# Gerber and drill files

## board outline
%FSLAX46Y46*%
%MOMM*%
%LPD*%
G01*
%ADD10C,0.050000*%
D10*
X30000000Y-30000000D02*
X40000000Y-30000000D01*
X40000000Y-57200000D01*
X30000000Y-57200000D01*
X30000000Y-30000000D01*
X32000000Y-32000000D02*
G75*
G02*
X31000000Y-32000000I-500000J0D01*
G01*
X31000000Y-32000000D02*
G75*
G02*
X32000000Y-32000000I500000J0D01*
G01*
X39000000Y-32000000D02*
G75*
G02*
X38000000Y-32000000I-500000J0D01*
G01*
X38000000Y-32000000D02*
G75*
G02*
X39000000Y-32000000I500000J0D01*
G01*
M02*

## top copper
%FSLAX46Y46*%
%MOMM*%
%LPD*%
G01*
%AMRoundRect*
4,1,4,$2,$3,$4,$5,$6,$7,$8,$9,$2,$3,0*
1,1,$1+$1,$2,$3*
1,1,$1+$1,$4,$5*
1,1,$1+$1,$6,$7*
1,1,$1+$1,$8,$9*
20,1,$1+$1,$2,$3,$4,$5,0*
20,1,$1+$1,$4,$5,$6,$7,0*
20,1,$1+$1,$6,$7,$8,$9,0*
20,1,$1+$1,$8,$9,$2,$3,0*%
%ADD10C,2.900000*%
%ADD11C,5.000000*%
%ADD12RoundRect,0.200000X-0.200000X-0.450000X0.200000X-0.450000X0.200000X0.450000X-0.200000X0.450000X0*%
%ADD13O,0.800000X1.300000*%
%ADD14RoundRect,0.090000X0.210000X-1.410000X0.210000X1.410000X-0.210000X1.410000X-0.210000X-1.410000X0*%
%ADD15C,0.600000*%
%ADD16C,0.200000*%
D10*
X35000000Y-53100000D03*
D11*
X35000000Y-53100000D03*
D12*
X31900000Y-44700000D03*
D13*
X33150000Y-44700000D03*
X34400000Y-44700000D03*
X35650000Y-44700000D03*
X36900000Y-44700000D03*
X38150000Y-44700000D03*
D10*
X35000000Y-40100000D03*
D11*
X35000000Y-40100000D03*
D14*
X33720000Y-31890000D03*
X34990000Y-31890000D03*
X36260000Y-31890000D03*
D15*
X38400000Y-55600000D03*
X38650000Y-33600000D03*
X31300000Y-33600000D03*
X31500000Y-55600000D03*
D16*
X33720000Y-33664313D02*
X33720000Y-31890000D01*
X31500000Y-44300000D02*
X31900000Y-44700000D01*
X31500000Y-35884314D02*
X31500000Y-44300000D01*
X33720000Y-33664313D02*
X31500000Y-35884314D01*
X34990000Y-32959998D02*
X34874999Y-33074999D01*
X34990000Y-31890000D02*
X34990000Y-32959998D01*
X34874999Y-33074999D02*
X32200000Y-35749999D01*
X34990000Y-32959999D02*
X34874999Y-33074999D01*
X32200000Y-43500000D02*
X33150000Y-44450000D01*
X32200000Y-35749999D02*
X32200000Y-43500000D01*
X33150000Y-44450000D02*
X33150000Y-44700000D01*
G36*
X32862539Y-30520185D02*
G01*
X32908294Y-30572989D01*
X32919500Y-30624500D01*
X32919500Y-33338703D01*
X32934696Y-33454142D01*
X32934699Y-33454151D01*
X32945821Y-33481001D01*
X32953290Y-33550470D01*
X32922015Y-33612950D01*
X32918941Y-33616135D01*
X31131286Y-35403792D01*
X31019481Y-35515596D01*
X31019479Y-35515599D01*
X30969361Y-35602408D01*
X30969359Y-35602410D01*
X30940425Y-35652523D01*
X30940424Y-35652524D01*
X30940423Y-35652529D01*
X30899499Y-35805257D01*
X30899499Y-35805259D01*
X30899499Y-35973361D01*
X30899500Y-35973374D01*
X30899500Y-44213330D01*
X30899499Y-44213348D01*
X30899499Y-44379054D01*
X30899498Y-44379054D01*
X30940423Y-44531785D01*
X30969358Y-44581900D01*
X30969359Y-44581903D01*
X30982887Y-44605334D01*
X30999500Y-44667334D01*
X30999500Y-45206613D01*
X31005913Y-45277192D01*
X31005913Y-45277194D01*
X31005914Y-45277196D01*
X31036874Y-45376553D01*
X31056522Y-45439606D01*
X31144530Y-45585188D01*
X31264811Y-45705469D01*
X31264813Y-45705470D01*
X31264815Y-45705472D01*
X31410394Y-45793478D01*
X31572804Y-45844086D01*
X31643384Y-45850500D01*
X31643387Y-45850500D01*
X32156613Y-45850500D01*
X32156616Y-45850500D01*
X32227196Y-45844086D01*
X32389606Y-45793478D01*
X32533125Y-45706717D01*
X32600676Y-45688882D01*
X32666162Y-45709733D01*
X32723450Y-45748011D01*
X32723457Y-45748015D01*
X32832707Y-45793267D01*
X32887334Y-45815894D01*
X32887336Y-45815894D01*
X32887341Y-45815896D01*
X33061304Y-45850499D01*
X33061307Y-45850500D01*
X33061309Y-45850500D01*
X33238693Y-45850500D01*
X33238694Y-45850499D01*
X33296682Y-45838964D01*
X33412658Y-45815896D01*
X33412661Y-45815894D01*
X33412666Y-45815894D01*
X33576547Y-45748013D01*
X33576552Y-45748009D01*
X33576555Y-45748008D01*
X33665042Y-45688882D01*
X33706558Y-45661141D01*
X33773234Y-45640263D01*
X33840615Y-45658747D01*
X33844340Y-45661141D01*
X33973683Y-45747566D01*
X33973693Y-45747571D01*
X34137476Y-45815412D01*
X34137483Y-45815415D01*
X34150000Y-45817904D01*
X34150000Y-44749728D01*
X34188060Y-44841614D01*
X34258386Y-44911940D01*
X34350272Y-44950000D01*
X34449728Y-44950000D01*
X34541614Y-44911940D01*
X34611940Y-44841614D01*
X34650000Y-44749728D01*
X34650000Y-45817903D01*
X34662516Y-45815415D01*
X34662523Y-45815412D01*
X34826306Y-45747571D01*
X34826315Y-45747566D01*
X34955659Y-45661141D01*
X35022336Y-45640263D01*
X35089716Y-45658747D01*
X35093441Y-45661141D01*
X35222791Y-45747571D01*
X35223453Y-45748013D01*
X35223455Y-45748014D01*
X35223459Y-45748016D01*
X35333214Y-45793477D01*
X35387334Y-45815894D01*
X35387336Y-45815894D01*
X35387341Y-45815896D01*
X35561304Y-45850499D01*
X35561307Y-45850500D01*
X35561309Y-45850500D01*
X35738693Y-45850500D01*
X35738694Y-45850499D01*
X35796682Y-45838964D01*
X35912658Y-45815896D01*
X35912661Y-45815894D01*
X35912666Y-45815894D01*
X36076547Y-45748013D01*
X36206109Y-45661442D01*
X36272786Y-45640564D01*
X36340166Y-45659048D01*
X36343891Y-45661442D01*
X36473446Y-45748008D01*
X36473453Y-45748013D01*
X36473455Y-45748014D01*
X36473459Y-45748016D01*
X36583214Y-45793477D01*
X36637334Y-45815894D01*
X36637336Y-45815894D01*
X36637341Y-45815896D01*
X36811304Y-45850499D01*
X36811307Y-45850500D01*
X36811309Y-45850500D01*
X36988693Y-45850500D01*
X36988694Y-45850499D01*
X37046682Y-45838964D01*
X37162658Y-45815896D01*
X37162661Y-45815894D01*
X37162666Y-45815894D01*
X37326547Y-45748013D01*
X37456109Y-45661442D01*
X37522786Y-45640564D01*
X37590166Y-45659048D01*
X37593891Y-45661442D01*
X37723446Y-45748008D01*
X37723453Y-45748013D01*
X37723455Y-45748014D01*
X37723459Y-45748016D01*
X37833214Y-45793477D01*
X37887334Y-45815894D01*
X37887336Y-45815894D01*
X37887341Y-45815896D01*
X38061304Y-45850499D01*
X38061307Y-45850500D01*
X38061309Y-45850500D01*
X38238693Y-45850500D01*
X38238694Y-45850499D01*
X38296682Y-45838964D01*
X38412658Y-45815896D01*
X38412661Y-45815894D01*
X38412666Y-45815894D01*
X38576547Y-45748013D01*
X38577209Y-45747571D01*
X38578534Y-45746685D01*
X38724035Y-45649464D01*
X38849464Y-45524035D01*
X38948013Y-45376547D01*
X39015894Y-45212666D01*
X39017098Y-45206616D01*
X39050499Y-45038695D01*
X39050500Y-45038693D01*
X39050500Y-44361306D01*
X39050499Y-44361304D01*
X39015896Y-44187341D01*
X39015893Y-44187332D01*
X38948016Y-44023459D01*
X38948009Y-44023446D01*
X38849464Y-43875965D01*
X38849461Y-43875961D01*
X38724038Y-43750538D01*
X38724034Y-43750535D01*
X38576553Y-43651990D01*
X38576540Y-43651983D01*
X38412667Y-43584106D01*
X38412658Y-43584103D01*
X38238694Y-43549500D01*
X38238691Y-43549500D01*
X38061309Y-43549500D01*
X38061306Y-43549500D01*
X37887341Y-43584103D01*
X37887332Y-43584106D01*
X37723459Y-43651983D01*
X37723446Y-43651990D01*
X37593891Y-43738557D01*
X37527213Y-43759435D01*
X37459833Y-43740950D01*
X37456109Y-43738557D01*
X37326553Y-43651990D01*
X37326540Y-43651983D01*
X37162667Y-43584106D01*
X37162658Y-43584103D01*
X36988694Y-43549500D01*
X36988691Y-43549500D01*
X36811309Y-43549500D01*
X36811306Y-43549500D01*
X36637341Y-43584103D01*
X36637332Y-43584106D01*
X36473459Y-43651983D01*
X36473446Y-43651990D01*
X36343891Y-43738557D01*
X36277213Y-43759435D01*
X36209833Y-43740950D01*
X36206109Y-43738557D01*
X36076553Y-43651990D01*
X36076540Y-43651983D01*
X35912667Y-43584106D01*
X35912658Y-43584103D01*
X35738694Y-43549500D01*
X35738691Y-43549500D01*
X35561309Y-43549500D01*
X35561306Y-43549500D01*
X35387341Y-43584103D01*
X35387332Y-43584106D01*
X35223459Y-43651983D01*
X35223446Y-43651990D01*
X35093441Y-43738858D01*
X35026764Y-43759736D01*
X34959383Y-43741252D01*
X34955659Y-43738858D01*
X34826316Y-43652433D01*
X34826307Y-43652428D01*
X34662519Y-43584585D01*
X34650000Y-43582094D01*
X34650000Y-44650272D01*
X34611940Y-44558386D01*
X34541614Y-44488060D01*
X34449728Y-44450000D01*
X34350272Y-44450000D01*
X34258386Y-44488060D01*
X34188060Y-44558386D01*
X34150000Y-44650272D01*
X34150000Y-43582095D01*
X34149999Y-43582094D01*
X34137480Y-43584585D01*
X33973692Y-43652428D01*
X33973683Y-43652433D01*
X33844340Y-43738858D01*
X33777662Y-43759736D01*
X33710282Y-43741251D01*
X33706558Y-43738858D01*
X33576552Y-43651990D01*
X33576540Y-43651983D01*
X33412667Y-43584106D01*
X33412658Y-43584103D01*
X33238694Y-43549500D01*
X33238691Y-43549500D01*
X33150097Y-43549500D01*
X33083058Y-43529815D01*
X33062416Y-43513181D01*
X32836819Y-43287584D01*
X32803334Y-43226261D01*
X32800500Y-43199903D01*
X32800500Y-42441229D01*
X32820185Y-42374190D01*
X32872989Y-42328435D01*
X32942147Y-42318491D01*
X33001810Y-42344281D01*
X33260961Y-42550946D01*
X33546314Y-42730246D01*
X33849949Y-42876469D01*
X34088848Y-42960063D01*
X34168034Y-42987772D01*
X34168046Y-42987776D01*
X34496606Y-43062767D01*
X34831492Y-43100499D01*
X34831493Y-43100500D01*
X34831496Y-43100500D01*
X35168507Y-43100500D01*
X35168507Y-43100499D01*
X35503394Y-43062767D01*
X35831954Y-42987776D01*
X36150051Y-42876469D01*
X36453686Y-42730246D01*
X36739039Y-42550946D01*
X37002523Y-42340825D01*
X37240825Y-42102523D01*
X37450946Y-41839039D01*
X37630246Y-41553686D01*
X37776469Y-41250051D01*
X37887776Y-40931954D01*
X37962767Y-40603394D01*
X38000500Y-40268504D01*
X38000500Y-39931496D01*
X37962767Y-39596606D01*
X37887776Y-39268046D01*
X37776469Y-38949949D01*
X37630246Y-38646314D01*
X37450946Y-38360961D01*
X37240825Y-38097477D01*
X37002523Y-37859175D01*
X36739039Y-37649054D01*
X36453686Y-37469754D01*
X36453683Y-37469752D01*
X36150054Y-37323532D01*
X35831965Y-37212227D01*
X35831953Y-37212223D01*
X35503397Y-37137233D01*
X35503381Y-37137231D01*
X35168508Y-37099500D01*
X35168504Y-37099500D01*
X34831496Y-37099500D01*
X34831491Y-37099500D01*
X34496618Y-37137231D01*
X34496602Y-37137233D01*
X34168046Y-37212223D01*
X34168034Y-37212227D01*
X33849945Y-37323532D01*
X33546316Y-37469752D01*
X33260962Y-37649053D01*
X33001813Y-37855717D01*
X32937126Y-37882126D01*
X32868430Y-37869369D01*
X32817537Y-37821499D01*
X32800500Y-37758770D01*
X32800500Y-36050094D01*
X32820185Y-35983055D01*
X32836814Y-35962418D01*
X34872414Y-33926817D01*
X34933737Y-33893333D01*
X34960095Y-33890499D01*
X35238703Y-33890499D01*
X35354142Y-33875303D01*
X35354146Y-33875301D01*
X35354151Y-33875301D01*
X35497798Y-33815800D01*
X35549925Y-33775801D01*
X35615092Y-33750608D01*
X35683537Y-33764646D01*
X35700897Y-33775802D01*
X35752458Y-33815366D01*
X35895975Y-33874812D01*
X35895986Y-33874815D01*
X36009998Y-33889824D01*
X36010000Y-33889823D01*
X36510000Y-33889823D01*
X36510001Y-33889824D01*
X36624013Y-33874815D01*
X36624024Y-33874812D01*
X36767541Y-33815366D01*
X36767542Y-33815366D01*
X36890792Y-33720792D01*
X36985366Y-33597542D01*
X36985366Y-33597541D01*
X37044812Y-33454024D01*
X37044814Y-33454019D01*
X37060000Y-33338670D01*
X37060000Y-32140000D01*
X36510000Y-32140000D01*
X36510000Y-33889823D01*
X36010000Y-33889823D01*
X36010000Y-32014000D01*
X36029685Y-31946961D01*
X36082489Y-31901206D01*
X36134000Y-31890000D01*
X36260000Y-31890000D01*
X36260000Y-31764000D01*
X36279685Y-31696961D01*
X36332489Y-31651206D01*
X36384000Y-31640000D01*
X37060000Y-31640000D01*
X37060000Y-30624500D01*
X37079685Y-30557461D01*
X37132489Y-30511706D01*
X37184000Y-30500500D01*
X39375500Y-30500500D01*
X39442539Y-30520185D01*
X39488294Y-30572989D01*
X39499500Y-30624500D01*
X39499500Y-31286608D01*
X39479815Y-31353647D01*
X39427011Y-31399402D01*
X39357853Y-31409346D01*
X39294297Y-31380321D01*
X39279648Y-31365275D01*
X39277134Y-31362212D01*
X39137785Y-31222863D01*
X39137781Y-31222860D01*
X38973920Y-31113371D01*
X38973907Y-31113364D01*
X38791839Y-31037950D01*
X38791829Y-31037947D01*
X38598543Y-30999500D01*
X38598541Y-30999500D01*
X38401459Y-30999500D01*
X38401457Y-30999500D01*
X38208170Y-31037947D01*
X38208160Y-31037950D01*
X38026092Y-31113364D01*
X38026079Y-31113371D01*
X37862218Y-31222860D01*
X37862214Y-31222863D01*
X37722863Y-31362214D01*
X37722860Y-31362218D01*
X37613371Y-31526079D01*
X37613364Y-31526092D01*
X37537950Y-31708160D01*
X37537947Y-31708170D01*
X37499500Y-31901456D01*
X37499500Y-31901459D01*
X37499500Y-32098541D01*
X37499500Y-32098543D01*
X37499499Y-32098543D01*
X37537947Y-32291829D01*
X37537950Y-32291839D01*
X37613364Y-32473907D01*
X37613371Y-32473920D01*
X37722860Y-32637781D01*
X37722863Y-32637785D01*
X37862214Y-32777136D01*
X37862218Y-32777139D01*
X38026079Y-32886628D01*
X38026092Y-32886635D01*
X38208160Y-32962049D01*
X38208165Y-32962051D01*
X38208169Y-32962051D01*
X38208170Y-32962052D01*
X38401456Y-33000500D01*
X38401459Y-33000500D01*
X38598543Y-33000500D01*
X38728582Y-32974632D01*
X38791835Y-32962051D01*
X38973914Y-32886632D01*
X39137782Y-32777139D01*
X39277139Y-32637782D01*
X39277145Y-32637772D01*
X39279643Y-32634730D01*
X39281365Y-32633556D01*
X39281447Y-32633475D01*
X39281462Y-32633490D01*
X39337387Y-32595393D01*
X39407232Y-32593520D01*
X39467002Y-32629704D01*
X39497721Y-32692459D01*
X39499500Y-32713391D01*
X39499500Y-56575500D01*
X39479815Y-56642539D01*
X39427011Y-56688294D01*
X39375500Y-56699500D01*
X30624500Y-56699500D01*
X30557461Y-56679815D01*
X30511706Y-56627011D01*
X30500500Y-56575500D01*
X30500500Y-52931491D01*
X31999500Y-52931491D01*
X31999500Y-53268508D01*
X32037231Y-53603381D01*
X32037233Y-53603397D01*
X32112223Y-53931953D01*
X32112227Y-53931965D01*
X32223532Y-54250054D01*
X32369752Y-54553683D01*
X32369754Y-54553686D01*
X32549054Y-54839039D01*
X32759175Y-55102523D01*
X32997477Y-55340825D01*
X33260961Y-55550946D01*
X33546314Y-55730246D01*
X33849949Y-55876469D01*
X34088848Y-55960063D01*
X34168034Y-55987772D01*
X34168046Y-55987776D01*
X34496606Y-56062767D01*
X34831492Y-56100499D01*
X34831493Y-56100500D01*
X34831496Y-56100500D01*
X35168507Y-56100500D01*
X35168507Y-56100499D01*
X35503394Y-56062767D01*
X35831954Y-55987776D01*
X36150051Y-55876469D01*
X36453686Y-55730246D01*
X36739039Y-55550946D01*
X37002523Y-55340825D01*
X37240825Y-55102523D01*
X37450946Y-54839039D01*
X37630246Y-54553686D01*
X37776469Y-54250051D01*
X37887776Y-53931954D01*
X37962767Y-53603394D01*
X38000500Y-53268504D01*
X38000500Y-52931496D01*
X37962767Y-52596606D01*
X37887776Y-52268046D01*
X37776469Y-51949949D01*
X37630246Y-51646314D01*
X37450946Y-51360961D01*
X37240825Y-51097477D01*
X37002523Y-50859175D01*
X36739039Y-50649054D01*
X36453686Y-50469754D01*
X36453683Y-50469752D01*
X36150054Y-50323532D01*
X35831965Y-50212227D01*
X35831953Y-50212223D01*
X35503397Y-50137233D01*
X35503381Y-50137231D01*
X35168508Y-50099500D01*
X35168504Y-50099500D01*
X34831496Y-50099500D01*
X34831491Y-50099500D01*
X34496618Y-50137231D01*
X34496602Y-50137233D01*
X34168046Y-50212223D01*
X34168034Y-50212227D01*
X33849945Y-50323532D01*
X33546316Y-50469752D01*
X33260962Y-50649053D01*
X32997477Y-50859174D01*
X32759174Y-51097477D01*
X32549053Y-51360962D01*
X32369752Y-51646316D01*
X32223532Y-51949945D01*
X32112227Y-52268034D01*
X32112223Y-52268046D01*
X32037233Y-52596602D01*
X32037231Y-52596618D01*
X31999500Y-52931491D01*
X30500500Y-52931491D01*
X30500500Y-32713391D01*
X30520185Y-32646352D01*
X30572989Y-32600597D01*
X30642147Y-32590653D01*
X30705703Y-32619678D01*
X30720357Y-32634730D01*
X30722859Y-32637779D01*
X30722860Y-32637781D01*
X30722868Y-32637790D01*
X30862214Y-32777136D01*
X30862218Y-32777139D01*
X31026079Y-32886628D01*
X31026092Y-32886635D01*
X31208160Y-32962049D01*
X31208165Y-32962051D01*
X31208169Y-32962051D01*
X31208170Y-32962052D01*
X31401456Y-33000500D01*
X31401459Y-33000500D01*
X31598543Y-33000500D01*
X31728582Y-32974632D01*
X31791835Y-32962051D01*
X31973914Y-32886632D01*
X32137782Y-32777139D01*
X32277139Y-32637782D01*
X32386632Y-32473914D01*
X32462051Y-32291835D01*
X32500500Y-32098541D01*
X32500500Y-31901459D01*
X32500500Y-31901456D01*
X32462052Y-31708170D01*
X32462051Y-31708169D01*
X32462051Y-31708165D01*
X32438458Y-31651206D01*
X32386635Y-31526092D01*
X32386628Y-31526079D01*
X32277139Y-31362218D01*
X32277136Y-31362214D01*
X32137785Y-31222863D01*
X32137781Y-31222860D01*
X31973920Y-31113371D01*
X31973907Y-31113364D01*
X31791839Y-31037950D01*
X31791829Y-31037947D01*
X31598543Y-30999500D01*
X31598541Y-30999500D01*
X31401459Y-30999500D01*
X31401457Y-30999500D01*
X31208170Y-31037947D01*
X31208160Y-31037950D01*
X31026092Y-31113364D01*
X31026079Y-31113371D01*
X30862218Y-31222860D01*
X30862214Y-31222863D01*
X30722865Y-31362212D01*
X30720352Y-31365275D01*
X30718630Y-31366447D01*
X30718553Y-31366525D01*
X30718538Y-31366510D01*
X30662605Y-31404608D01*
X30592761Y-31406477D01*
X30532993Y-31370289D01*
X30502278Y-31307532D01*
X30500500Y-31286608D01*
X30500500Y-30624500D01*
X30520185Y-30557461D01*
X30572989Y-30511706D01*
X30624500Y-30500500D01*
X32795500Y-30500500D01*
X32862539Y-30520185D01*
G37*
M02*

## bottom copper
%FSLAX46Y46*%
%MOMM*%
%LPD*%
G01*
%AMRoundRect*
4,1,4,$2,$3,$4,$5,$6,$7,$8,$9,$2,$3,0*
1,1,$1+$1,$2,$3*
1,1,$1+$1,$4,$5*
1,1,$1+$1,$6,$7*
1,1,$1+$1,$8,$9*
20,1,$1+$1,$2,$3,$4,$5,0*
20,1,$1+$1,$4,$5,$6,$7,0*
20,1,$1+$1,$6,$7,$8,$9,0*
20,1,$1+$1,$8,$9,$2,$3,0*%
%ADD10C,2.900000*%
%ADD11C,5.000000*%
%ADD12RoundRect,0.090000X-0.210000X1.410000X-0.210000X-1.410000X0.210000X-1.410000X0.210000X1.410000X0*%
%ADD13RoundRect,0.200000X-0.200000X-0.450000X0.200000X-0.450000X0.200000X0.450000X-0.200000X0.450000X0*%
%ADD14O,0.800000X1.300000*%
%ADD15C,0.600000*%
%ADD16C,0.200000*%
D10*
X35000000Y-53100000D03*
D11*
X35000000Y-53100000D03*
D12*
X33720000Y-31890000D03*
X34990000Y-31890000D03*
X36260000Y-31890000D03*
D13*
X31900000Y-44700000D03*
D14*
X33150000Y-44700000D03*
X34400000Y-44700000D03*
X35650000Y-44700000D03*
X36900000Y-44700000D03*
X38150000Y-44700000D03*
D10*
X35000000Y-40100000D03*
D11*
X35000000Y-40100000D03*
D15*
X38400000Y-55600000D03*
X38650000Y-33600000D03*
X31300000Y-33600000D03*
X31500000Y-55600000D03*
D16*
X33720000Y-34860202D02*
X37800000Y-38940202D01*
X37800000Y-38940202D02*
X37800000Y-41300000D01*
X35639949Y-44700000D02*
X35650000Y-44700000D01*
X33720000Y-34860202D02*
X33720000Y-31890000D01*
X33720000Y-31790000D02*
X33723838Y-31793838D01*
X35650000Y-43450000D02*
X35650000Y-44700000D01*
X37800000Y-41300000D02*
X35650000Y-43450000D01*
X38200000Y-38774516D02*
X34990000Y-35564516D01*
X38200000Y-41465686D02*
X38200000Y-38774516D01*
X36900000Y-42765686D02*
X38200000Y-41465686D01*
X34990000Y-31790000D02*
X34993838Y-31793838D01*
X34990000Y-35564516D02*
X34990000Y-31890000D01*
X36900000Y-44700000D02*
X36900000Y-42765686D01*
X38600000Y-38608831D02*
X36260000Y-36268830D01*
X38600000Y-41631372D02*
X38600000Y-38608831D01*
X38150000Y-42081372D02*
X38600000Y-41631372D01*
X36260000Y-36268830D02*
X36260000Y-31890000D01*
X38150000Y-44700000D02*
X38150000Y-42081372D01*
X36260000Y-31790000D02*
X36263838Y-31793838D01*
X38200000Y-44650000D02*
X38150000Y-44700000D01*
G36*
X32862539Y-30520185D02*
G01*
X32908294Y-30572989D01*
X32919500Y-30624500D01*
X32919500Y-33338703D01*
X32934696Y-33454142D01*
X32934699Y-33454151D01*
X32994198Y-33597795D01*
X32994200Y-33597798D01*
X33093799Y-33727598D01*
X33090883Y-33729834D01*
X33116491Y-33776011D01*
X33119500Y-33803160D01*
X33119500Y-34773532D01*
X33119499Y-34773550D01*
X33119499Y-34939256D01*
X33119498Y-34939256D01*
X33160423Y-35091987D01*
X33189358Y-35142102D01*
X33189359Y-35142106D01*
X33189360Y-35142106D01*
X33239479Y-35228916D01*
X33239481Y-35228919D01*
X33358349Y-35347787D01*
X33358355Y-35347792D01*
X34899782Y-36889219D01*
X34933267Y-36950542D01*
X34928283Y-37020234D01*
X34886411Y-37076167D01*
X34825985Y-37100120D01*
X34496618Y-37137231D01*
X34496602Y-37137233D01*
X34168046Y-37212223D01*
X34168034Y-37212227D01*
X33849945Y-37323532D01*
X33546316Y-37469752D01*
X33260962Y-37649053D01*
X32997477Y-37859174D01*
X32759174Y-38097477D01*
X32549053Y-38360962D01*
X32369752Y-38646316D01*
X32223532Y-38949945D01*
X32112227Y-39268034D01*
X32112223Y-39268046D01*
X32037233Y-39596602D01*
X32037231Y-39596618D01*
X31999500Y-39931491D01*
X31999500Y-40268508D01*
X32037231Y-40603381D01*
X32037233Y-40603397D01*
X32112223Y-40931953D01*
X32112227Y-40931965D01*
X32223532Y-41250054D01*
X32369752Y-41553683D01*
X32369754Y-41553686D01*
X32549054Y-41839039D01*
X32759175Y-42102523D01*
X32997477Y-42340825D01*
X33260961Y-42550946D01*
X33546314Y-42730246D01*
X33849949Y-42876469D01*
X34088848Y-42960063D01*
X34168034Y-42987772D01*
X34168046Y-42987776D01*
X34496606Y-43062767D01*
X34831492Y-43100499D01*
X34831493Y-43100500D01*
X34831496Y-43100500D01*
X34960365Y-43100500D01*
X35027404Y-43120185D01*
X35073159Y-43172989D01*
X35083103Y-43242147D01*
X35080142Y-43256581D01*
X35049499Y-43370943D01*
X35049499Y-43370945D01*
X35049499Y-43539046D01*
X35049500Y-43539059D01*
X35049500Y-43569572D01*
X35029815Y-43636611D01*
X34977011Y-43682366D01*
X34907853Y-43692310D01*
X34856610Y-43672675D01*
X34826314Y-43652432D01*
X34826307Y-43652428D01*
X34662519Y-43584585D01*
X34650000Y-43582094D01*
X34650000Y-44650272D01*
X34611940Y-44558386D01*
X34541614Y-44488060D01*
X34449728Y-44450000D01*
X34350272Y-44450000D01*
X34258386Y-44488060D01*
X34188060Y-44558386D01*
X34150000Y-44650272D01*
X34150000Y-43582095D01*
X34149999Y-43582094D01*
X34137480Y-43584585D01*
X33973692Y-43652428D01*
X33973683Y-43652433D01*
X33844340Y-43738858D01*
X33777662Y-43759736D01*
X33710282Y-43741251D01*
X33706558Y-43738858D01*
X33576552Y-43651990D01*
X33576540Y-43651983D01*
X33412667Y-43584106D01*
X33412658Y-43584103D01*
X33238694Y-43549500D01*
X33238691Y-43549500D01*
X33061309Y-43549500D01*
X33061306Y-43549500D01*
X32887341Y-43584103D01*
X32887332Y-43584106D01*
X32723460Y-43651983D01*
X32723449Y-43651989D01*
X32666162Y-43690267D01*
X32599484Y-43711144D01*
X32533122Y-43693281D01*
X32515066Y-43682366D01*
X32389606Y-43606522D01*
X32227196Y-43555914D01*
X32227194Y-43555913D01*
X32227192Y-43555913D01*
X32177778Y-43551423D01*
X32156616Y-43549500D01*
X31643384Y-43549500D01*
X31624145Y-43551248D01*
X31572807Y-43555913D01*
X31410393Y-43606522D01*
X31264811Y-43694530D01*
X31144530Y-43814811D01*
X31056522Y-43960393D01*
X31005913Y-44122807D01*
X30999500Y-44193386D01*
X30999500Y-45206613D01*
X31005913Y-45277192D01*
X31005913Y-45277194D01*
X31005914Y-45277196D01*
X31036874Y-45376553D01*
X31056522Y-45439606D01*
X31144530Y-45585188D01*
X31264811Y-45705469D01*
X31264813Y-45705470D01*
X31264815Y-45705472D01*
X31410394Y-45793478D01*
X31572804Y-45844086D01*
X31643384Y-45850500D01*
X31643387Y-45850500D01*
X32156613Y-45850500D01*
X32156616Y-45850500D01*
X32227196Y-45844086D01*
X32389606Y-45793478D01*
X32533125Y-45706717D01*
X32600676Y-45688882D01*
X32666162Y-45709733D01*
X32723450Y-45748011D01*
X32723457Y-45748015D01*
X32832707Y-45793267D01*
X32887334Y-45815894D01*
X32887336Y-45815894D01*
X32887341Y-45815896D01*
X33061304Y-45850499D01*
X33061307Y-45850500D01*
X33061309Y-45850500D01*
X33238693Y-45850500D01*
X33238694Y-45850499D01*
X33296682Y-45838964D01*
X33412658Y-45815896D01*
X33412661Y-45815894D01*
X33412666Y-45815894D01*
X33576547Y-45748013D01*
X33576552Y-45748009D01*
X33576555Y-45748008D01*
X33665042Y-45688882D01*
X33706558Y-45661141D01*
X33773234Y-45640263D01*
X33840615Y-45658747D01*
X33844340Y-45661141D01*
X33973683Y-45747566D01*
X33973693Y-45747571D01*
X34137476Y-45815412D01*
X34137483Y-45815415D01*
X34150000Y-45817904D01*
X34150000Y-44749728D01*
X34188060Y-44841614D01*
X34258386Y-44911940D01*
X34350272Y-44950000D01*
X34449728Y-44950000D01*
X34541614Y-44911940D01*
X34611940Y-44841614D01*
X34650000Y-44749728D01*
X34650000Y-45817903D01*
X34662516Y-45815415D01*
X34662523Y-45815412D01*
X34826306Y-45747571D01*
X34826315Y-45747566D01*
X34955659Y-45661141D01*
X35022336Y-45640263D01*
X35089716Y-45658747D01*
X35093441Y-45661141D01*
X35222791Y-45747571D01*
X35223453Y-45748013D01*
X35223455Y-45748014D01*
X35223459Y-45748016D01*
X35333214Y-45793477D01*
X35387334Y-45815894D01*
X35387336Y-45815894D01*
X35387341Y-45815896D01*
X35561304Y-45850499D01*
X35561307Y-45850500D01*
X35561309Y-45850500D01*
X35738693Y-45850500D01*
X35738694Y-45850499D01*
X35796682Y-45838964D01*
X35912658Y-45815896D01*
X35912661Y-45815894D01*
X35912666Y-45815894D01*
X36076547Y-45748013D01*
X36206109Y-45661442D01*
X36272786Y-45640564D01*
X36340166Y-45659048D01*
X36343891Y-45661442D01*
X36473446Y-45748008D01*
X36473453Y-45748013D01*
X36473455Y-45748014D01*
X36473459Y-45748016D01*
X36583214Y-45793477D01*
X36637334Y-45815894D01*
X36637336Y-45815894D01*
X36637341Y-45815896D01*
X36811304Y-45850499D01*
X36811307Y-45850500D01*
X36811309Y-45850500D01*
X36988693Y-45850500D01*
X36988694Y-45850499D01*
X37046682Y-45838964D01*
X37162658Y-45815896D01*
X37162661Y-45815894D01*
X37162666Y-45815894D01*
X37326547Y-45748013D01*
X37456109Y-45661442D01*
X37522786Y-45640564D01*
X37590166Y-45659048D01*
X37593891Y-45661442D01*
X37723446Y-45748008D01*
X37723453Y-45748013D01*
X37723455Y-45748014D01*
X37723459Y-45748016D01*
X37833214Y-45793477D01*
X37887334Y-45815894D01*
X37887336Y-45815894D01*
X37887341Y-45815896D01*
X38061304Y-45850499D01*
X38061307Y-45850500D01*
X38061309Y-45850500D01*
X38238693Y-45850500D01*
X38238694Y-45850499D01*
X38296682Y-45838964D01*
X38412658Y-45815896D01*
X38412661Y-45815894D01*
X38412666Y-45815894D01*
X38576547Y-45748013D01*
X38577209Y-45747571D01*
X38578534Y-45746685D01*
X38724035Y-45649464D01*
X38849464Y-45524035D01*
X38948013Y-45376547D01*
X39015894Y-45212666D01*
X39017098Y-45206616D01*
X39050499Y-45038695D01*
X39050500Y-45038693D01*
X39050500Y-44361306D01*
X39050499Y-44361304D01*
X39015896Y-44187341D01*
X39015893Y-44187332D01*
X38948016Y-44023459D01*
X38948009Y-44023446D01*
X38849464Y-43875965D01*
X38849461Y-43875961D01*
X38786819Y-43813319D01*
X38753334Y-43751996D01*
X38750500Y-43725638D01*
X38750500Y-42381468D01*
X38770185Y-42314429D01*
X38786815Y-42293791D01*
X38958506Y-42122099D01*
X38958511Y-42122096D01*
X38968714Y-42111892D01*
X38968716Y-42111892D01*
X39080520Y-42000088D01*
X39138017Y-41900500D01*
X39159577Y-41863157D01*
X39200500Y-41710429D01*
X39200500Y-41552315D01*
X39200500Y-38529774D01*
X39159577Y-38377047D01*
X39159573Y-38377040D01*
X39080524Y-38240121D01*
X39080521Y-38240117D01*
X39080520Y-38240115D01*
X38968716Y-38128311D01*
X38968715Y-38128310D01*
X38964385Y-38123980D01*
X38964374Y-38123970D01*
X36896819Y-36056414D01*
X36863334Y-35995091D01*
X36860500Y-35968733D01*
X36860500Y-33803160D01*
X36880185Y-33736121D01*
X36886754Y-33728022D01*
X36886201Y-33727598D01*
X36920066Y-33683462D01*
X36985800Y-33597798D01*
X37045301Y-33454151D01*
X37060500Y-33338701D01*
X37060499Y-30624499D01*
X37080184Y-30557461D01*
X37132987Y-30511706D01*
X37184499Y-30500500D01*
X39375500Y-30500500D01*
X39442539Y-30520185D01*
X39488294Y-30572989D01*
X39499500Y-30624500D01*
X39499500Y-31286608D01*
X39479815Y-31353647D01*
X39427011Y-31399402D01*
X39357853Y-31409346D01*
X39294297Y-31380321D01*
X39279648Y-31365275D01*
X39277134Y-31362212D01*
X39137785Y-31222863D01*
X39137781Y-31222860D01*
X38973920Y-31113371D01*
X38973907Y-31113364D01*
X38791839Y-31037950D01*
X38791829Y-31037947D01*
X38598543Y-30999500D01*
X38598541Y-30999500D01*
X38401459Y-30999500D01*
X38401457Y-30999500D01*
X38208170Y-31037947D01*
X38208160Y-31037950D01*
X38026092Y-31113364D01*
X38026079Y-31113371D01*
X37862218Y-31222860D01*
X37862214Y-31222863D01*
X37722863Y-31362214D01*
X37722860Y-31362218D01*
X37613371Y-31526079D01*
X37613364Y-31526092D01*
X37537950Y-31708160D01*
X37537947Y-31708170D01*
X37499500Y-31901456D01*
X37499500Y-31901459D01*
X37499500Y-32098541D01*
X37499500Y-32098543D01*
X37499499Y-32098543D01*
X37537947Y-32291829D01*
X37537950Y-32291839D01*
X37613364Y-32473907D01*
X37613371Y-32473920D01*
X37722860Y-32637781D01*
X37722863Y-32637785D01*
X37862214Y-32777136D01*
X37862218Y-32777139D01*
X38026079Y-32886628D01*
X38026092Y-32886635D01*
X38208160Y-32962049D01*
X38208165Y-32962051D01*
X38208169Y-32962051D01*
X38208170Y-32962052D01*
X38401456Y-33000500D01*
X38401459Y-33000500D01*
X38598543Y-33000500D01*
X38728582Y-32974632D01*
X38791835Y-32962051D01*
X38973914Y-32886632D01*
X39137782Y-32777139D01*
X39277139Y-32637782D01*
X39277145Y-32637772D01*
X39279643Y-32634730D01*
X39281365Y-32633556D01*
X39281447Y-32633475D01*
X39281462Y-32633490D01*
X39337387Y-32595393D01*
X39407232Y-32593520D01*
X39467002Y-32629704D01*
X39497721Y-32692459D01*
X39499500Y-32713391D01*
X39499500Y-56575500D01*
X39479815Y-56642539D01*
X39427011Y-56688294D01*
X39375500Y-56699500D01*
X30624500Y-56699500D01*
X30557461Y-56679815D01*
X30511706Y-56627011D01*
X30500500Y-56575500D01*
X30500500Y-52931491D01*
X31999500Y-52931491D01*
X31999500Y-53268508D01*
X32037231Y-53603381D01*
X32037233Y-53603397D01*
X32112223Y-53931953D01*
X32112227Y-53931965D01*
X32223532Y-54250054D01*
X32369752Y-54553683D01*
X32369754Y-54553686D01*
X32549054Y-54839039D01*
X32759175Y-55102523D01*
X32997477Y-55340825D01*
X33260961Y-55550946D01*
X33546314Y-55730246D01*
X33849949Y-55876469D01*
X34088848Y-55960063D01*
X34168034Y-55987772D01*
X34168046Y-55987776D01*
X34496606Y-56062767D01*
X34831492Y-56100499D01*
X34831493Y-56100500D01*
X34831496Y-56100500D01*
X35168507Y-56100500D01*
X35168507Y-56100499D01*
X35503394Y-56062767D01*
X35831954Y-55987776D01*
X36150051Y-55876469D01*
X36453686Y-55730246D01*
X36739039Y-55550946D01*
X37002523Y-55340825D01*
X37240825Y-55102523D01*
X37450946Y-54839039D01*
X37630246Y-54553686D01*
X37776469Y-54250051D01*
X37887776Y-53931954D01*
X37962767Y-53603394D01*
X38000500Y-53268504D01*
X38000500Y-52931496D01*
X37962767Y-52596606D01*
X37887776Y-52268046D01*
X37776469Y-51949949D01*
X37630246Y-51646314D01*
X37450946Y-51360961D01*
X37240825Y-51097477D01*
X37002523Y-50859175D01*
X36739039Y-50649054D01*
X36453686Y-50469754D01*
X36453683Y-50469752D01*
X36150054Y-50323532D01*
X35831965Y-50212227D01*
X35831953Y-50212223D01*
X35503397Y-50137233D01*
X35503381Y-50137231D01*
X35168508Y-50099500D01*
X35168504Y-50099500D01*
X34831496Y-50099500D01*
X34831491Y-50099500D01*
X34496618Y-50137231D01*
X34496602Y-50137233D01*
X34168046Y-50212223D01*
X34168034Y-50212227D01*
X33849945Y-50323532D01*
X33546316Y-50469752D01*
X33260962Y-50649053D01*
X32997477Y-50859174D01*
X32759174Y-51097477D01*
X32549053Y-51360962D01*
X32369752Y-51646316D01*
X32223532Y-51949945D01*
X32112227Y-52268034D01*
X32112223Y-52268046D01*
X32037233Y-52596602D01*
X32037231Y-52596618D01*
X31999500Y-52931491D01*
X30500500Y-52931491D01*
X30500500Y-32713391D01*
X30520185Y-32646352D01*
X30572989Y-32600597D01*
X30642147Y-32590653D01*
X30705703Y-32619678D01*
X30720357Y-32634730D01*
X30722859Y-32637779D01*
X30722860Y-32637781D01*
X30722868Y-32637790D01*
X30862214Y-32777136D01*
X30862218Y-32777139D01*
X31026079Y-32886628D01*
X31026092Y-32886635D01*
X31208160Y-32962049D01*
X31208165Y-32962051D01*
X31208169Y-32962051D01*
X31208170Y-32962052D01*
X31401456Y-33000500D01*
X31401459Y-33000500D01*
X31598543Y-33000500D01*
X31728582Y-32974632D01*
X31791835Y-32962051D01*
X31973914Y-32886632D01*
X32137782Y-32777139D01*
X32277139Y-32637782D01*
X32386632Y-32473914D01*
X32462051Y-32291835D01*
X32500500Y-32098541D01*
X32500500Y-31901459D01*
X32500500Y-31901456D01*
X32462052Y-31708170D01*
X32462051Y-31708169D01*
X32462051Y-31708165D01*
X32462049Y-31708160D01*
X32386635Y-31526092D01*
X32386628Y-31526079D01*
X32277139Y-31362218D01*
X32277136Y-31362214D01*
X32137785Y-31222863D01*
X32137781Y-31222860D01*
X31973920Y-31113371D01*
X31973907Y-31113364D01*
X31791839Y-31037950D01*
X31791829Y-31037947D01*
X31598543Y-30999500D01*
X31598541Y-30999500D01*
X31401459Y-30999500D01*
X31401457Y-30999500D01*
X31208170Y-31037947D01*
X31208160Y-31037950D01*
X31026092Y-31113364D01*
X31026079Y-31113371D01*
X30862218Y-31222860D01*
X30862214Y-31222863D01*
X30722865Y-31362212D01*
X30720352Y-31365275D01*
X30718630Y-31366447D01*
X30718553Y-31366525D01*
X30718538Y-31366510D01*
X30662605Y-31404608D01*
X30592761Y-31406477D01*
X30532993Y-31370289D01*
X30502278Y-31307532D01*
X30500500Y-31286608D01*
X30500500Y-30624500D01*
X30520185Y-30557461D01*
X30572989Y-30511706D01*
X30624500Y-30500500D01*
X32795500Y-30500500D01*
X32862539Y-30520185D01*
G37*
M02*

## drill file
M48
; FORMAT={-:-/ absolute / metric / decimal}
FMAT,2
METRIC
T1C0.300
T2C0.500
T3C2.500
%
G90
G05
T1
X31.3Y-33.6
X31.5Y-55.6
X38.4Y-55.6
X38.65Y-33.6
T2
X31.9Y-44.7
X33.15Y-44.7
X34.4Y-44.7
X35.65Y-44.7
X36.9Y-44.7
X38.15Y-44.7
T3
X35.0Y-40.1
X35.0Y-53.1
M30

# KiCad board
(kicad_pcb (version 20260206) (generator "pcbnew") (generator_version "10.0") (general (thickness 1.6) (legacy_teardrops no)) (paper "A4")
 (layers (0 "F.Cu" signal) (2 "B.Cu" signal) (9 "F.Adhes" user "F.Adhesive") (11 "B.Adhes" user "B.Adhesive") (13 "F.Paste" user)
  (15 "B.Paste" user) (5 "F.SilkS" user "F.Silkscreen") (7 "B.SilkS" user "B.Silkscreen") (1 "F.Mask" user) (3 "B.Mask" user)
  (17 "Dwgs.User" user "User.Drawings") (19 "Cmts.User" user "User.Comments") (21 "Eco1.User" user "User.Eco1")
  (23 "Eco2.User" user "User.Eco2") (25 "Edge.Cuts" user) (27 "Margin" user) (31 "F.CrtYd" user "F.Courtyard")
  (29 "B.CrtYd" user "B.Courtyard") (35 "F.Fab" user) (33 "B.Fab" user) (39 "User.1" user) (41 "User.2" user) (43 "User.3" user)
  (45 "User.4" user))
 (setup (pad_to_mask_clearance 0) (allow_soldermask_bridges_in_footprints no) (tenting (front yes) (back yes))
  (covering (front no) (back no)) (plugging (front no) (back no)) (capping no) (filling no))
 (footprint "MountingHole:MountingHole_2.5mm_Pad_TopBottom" (layer "F.Cu") (at 35 53.1)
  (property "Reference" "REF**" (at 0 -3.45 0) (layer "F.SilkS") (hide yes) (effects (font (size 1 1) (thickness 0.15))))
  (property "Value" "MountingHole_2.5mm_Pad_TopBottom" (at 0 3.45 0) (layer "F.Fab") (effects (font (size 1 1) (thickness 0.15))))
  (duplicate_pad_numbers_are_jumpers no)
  (pad "1" thru_hole circle (at 0 0) (size 2.9 2.9) (drill 2.5) (layers "*.Cu" "*.Mask") (remove_unused_layers no) (zone_connect 2))
  (pad "1" connect circle (at 0 0) (size 5 5) (layers "F.Cu" "F.Mask") (zone_connect 2))
  (pad "1" connect circle (at 0 0) (size 5 5) (layers "B.Cu" "B.Mask") (zone_connect 2)))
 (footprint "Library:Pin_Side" (layer "F.Cu") (at 34.99 31.89 -90)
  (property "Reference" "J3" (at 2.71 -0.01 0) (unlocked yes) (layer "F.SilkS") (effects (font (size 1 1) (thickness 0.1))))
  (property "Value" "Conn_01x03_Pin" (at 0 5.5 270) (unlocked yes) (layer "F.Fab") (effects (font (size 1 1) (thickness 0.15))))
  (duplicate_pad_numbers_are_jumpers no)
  (pad "1" smd roundrect (at 0 1.27 270) (size 3 0.6) (layers "*.Mask" "B.Cu") (roundrect_rratio 0.15) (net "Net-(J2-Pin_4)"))
  (pad "2" smd roundrect (at 0 0 270) (size 3 0.6) (layers "*.Mask" "B.Cu") (roundrect_rratio 0.15) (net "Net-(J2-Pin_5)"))
  (pad "3" smd roundrect (at 0 -1.27 270) (size 3 0.6) (layers "*.Mask" "B.Cu") (roundrect_rratio 0.15) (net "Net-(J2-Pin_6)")))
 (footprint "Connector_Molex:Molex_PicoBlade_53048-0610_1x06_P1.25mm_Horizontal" (layer "F.Cu") (at 31.9 44.7)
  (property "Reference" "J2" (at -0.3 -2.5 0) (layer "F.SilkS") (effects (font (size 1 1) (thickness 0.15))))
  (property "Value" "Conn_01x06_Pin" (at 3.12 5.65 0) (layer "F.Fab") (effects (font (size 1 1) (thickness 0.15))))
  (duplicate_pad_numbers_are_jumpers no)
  (pad "1" thru_hole roundrect (at 0 0) (size 0.8 1.3) (drill 0.5) (layers "*.Cu" "*.Mask") (remove_unused_layers no)
   (roundrect_rratio 0.25) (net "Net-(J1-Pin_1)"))
  (pad "2" thru_hole oval (at 1.25 0) (size 0.8 1.3) (drill 0.5) (layers "*.Cu" "*.Mask") (remove_unused_layers no) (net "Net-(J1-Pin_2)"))
  (pad "3" thru_hole oval (at 2.5 0) (size 0.8 1.3) (drill 0.5) (layers "*.Cu" "*.Mask") (remove_unused_layers no) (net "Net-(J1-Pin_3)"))
  (pad "4" thru_hole oval (at 3.75 0) (size 0.8 1.3) (drill 0.5) (layers "*.Cu" "*.Mask") (remove_unused_layers no) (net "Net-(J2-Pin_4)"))
  (pad "5" thru_hole oval (at 5 0) (size 0.8 1.3) (drill 0.5) (layers "*.Cu" "*.Mask") (remove_unused_layers no) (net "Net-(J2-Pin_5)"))
  (pad "6" thru_hole oval (at 6.25 0) (size 0.8 1.3) (drill 0.5) (layers "*.Cu" "*.Mask") (remove_unused_layers no) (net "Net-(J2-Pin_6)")))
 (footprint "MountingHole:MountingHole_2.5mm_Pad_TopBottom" (layer "F.Cu") (at 35 40.1)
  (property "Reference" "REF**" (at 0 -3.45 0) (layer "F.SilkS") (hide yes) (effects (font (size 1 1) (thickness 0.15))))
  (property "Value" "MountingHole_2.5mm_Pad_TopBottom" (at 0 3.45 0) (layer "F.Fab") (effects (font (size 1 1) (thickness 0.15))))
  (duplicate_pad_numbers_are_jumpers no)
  (pad "1" thru_hole circle (at 0 0) (size 2.9 2.9) (drill 2.5) (layers "*.Cu" "*.Mask") (remove_unused_layers no) (zone_connect 2))
  (pad "1" connect circle (at 0 0) (size 5 5) (layers "F.Cu" "F.Mask") (zone_connect 2))
  (pad "1" connect circle (at 0 0) (size 5 5) (layers "B.Cu" "B.Mask") (zone_connect 2)))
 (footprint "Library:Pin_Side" (layer "B.Cu") (at 34.99 31.89 90)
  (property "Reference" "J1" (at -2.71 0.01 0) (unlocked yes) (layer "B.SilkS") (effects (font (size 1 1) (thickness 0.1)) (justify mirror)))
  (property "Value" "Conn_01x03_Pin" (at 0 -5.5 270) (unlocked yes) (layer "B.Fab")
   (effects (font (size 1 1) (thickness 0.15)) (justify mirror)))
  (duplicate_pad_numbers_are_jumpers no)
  (pad "1" smd roundrect (at 0 -1.27 90) (size 3 0.6) (layers "*.Mask" "F.Cu") (roundrect_rratio 0.15) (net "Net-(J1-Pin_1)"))
  (pad "2" smd roundrect (at 0 0 90) (size 3 0.6) (layers "*.Mask" "F.Cu") (roundrect_rratio 0.15) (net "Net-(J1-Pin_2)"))
  (pad "3" smd roundrect (at 0 1.27 90) (size 3 0.6) (layers "*.Mask" "F.Cu") (roundrect_rratio 0.15) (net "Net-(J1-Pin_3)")))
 (gr_rect (start 30 30) (end 40 57.2) (stroke (width 0.05) (type default)) (fill no) (layer "Edge.Cuts"))
 (gr_circle (center 31.5 32) (end 31 32) (stroke (width 0.05) (type default)) (fill no) (layer "Edge.Cuts"))
 (gr_circle (center 38.5 32) (end 39 32) (stroke (width 0.05) (type default)) (fill no) (layer "Edge.Cuts"))
 (segment (start 33.72 34.860202) (end 37.8 38.940202) (width 0.2) (layer "B.Cu") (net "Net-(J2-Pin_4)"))
 (segment (start 37.8 38.940202) (end 37.8 41.3) (width 0.2) (layer "B.Cu") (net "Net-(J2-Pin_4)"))
 (segment (start 35.639949 44.7) (end 35.65 44.7) (width 0.2) (layer "B.Cu") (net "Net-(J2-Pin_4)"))
 (segment (start 33.72 34.860202) (end 33.72 31.89) (width 0.2) (layer "B.Cu") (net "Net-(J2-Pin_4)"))
 (segment (start 33.72 31.79) (end 33.723838 31.793838) (width 0.2) (layer "B.Cu") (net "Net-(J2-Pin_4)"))
 (segment (start 35.65 43.45) (end 35.65 44.7) (width 0.2) (layer "B.Cu") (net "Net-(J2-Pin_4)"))
 (segment (start 37.8 41.3) (end 35.65 43.45) (width 0.2) (layer "B.Cu") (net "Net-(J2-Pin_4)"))
 (segment (start 38.2 38.774516) (end 34.99 35.564516) (width 0.2) (layer "B.Cu") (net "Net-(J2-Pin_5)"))
 (segment (start 38.2 41.465686) (end 38.2 38.774516) (width 0.2) (layer "B.Cu") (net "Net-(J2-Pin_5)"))
 (segment (start 36.9 42.765686) (end 38.2 41.465686) (width 0.2) (layer "B.Cu") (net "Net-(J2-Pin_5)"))
 (segment (start 34.99 31.79) (end 34.993838 31.793838) (width 0.2) (layer "B.Cu") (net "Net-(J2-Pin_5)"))
 (segment (start 34.99 35.564516) (end 34.99 31.89) (width 0.2) (layer "B.Cu") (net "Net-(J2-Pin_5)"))
 (segment (start 36.9 44.7) (end 36.9 42.765686) (width 0.2) (layer "B.Cu") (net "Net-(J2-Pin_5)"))
 (segment (start 38.6 38.608831) (end 36.26 36.26883) (width 0.2) (layer "B.Cu") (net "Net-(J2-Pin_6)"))
 (segment (start 38.6 41.631372) (end 38.6 38.608831) (width 0.2) (layer "B.Cu") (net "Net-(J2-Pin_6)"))
 (segment (start 38.15 42.081372) (end 38.6 41.631372) (width 0.2) (layer "B.Cu") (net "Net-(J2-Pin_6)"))
 (segment (start 36.26 36.26883) (end 36.26 31.89) (width 0.2) (layer "B.Cu") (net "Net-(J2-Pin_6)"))
 (segment (start 38.15 44.7) (end 38.15 42.081372) (width 0.2) (layer "B.Cu") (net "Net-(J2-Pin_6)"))
 (segment (start 36.26 31.79) (end 36.263838 31.793838) (width 0.2) (layer "B.Cu") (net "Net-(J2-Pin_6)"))
 (segment (start 38.2 44.65) (end 38.15 44.7) (width 0.2) (layer "B.Cu") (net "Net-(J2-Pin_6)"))
 (segment (start 33.72 33.664313) (end 33.72 31.89) (width 0.2) (layer "F.Cu") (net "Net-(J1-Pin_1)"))
 (segment (start 31.5 44.3) (end 31.9 44.7) (width 0.2) (layer "F.Cu") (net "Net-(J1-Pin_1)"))
 (segment (start 31.5 35.884314) (end 31.5 44.3) (width 0.2) (layer "F.Cu") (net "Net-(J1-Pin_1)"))
 (segment (start 33.72 33.664313) (end 31.5 35.884314) (width 0.2) (layer "F.Cu") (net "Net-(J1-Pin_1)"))
 (segment (start 34.99 32.959998) (end 34.874999 33.074999) (width 0.2) (layer "F.Cu") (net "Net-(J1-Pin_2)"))
 (segment (start 34.99 31.89) (end 34.99 32.959998) (width 0.2) (layer "F.Cu") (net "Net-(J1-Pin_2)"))
 (segment (start 34.874999 33.074999) (end 32.2 35.749999) (width 0.2) (layer "F.Cu") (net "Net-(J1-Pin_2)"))
 (segment (start 34.99 32.959999) (end 34.874999 33.074999) (width 0.2) (layer "F.Cu") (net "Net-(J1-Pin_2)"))
 (segment (start 32.2 43.5) (end 33.15 44.45) (width 0.2) (layer "F.Cu") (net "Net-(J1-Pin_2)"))
 (segment (start 32.2 35.749999) (end 32.2 43.5) (width 0.2) (layer "F.Cu") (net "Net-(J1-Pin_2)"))
 (segment (start 33.15 44.45) (end 33.15 44.7) (width 0.2) (layer "F.Cu") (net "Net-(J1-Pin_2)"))
 (via (at 38.4 55.6) (size 0.6) (drill 0.3) (layers "F.Cu" "B.Cu") (free yes) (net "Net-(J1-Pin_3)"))
 (via (at 38.65 33.6) (size 0.6) (drill 0.3) (layers "F.Cu" "B.Cu") (free yes) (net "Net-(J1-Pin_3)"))
 (via (at 31.3 33.6) (size 0.6) (drill 0.3) (layers "F.Cu" "B.Cu") (free yes) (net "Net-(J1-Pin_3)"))
 (via (at 31.5 55.6) (size 0.6) (drill 0.3) (layers "F.Cu" "B.Cu") (free yes) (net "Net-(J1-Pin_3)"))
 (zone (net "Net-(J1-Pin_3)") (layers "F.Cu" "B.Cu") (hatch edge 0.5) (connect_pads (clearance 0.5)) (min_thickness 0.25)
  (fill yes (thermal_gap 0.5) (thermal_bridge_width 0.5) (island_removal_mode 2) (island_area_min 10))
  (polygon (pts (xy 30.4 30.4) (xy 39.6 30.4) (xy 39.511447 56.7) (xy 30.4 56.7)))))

